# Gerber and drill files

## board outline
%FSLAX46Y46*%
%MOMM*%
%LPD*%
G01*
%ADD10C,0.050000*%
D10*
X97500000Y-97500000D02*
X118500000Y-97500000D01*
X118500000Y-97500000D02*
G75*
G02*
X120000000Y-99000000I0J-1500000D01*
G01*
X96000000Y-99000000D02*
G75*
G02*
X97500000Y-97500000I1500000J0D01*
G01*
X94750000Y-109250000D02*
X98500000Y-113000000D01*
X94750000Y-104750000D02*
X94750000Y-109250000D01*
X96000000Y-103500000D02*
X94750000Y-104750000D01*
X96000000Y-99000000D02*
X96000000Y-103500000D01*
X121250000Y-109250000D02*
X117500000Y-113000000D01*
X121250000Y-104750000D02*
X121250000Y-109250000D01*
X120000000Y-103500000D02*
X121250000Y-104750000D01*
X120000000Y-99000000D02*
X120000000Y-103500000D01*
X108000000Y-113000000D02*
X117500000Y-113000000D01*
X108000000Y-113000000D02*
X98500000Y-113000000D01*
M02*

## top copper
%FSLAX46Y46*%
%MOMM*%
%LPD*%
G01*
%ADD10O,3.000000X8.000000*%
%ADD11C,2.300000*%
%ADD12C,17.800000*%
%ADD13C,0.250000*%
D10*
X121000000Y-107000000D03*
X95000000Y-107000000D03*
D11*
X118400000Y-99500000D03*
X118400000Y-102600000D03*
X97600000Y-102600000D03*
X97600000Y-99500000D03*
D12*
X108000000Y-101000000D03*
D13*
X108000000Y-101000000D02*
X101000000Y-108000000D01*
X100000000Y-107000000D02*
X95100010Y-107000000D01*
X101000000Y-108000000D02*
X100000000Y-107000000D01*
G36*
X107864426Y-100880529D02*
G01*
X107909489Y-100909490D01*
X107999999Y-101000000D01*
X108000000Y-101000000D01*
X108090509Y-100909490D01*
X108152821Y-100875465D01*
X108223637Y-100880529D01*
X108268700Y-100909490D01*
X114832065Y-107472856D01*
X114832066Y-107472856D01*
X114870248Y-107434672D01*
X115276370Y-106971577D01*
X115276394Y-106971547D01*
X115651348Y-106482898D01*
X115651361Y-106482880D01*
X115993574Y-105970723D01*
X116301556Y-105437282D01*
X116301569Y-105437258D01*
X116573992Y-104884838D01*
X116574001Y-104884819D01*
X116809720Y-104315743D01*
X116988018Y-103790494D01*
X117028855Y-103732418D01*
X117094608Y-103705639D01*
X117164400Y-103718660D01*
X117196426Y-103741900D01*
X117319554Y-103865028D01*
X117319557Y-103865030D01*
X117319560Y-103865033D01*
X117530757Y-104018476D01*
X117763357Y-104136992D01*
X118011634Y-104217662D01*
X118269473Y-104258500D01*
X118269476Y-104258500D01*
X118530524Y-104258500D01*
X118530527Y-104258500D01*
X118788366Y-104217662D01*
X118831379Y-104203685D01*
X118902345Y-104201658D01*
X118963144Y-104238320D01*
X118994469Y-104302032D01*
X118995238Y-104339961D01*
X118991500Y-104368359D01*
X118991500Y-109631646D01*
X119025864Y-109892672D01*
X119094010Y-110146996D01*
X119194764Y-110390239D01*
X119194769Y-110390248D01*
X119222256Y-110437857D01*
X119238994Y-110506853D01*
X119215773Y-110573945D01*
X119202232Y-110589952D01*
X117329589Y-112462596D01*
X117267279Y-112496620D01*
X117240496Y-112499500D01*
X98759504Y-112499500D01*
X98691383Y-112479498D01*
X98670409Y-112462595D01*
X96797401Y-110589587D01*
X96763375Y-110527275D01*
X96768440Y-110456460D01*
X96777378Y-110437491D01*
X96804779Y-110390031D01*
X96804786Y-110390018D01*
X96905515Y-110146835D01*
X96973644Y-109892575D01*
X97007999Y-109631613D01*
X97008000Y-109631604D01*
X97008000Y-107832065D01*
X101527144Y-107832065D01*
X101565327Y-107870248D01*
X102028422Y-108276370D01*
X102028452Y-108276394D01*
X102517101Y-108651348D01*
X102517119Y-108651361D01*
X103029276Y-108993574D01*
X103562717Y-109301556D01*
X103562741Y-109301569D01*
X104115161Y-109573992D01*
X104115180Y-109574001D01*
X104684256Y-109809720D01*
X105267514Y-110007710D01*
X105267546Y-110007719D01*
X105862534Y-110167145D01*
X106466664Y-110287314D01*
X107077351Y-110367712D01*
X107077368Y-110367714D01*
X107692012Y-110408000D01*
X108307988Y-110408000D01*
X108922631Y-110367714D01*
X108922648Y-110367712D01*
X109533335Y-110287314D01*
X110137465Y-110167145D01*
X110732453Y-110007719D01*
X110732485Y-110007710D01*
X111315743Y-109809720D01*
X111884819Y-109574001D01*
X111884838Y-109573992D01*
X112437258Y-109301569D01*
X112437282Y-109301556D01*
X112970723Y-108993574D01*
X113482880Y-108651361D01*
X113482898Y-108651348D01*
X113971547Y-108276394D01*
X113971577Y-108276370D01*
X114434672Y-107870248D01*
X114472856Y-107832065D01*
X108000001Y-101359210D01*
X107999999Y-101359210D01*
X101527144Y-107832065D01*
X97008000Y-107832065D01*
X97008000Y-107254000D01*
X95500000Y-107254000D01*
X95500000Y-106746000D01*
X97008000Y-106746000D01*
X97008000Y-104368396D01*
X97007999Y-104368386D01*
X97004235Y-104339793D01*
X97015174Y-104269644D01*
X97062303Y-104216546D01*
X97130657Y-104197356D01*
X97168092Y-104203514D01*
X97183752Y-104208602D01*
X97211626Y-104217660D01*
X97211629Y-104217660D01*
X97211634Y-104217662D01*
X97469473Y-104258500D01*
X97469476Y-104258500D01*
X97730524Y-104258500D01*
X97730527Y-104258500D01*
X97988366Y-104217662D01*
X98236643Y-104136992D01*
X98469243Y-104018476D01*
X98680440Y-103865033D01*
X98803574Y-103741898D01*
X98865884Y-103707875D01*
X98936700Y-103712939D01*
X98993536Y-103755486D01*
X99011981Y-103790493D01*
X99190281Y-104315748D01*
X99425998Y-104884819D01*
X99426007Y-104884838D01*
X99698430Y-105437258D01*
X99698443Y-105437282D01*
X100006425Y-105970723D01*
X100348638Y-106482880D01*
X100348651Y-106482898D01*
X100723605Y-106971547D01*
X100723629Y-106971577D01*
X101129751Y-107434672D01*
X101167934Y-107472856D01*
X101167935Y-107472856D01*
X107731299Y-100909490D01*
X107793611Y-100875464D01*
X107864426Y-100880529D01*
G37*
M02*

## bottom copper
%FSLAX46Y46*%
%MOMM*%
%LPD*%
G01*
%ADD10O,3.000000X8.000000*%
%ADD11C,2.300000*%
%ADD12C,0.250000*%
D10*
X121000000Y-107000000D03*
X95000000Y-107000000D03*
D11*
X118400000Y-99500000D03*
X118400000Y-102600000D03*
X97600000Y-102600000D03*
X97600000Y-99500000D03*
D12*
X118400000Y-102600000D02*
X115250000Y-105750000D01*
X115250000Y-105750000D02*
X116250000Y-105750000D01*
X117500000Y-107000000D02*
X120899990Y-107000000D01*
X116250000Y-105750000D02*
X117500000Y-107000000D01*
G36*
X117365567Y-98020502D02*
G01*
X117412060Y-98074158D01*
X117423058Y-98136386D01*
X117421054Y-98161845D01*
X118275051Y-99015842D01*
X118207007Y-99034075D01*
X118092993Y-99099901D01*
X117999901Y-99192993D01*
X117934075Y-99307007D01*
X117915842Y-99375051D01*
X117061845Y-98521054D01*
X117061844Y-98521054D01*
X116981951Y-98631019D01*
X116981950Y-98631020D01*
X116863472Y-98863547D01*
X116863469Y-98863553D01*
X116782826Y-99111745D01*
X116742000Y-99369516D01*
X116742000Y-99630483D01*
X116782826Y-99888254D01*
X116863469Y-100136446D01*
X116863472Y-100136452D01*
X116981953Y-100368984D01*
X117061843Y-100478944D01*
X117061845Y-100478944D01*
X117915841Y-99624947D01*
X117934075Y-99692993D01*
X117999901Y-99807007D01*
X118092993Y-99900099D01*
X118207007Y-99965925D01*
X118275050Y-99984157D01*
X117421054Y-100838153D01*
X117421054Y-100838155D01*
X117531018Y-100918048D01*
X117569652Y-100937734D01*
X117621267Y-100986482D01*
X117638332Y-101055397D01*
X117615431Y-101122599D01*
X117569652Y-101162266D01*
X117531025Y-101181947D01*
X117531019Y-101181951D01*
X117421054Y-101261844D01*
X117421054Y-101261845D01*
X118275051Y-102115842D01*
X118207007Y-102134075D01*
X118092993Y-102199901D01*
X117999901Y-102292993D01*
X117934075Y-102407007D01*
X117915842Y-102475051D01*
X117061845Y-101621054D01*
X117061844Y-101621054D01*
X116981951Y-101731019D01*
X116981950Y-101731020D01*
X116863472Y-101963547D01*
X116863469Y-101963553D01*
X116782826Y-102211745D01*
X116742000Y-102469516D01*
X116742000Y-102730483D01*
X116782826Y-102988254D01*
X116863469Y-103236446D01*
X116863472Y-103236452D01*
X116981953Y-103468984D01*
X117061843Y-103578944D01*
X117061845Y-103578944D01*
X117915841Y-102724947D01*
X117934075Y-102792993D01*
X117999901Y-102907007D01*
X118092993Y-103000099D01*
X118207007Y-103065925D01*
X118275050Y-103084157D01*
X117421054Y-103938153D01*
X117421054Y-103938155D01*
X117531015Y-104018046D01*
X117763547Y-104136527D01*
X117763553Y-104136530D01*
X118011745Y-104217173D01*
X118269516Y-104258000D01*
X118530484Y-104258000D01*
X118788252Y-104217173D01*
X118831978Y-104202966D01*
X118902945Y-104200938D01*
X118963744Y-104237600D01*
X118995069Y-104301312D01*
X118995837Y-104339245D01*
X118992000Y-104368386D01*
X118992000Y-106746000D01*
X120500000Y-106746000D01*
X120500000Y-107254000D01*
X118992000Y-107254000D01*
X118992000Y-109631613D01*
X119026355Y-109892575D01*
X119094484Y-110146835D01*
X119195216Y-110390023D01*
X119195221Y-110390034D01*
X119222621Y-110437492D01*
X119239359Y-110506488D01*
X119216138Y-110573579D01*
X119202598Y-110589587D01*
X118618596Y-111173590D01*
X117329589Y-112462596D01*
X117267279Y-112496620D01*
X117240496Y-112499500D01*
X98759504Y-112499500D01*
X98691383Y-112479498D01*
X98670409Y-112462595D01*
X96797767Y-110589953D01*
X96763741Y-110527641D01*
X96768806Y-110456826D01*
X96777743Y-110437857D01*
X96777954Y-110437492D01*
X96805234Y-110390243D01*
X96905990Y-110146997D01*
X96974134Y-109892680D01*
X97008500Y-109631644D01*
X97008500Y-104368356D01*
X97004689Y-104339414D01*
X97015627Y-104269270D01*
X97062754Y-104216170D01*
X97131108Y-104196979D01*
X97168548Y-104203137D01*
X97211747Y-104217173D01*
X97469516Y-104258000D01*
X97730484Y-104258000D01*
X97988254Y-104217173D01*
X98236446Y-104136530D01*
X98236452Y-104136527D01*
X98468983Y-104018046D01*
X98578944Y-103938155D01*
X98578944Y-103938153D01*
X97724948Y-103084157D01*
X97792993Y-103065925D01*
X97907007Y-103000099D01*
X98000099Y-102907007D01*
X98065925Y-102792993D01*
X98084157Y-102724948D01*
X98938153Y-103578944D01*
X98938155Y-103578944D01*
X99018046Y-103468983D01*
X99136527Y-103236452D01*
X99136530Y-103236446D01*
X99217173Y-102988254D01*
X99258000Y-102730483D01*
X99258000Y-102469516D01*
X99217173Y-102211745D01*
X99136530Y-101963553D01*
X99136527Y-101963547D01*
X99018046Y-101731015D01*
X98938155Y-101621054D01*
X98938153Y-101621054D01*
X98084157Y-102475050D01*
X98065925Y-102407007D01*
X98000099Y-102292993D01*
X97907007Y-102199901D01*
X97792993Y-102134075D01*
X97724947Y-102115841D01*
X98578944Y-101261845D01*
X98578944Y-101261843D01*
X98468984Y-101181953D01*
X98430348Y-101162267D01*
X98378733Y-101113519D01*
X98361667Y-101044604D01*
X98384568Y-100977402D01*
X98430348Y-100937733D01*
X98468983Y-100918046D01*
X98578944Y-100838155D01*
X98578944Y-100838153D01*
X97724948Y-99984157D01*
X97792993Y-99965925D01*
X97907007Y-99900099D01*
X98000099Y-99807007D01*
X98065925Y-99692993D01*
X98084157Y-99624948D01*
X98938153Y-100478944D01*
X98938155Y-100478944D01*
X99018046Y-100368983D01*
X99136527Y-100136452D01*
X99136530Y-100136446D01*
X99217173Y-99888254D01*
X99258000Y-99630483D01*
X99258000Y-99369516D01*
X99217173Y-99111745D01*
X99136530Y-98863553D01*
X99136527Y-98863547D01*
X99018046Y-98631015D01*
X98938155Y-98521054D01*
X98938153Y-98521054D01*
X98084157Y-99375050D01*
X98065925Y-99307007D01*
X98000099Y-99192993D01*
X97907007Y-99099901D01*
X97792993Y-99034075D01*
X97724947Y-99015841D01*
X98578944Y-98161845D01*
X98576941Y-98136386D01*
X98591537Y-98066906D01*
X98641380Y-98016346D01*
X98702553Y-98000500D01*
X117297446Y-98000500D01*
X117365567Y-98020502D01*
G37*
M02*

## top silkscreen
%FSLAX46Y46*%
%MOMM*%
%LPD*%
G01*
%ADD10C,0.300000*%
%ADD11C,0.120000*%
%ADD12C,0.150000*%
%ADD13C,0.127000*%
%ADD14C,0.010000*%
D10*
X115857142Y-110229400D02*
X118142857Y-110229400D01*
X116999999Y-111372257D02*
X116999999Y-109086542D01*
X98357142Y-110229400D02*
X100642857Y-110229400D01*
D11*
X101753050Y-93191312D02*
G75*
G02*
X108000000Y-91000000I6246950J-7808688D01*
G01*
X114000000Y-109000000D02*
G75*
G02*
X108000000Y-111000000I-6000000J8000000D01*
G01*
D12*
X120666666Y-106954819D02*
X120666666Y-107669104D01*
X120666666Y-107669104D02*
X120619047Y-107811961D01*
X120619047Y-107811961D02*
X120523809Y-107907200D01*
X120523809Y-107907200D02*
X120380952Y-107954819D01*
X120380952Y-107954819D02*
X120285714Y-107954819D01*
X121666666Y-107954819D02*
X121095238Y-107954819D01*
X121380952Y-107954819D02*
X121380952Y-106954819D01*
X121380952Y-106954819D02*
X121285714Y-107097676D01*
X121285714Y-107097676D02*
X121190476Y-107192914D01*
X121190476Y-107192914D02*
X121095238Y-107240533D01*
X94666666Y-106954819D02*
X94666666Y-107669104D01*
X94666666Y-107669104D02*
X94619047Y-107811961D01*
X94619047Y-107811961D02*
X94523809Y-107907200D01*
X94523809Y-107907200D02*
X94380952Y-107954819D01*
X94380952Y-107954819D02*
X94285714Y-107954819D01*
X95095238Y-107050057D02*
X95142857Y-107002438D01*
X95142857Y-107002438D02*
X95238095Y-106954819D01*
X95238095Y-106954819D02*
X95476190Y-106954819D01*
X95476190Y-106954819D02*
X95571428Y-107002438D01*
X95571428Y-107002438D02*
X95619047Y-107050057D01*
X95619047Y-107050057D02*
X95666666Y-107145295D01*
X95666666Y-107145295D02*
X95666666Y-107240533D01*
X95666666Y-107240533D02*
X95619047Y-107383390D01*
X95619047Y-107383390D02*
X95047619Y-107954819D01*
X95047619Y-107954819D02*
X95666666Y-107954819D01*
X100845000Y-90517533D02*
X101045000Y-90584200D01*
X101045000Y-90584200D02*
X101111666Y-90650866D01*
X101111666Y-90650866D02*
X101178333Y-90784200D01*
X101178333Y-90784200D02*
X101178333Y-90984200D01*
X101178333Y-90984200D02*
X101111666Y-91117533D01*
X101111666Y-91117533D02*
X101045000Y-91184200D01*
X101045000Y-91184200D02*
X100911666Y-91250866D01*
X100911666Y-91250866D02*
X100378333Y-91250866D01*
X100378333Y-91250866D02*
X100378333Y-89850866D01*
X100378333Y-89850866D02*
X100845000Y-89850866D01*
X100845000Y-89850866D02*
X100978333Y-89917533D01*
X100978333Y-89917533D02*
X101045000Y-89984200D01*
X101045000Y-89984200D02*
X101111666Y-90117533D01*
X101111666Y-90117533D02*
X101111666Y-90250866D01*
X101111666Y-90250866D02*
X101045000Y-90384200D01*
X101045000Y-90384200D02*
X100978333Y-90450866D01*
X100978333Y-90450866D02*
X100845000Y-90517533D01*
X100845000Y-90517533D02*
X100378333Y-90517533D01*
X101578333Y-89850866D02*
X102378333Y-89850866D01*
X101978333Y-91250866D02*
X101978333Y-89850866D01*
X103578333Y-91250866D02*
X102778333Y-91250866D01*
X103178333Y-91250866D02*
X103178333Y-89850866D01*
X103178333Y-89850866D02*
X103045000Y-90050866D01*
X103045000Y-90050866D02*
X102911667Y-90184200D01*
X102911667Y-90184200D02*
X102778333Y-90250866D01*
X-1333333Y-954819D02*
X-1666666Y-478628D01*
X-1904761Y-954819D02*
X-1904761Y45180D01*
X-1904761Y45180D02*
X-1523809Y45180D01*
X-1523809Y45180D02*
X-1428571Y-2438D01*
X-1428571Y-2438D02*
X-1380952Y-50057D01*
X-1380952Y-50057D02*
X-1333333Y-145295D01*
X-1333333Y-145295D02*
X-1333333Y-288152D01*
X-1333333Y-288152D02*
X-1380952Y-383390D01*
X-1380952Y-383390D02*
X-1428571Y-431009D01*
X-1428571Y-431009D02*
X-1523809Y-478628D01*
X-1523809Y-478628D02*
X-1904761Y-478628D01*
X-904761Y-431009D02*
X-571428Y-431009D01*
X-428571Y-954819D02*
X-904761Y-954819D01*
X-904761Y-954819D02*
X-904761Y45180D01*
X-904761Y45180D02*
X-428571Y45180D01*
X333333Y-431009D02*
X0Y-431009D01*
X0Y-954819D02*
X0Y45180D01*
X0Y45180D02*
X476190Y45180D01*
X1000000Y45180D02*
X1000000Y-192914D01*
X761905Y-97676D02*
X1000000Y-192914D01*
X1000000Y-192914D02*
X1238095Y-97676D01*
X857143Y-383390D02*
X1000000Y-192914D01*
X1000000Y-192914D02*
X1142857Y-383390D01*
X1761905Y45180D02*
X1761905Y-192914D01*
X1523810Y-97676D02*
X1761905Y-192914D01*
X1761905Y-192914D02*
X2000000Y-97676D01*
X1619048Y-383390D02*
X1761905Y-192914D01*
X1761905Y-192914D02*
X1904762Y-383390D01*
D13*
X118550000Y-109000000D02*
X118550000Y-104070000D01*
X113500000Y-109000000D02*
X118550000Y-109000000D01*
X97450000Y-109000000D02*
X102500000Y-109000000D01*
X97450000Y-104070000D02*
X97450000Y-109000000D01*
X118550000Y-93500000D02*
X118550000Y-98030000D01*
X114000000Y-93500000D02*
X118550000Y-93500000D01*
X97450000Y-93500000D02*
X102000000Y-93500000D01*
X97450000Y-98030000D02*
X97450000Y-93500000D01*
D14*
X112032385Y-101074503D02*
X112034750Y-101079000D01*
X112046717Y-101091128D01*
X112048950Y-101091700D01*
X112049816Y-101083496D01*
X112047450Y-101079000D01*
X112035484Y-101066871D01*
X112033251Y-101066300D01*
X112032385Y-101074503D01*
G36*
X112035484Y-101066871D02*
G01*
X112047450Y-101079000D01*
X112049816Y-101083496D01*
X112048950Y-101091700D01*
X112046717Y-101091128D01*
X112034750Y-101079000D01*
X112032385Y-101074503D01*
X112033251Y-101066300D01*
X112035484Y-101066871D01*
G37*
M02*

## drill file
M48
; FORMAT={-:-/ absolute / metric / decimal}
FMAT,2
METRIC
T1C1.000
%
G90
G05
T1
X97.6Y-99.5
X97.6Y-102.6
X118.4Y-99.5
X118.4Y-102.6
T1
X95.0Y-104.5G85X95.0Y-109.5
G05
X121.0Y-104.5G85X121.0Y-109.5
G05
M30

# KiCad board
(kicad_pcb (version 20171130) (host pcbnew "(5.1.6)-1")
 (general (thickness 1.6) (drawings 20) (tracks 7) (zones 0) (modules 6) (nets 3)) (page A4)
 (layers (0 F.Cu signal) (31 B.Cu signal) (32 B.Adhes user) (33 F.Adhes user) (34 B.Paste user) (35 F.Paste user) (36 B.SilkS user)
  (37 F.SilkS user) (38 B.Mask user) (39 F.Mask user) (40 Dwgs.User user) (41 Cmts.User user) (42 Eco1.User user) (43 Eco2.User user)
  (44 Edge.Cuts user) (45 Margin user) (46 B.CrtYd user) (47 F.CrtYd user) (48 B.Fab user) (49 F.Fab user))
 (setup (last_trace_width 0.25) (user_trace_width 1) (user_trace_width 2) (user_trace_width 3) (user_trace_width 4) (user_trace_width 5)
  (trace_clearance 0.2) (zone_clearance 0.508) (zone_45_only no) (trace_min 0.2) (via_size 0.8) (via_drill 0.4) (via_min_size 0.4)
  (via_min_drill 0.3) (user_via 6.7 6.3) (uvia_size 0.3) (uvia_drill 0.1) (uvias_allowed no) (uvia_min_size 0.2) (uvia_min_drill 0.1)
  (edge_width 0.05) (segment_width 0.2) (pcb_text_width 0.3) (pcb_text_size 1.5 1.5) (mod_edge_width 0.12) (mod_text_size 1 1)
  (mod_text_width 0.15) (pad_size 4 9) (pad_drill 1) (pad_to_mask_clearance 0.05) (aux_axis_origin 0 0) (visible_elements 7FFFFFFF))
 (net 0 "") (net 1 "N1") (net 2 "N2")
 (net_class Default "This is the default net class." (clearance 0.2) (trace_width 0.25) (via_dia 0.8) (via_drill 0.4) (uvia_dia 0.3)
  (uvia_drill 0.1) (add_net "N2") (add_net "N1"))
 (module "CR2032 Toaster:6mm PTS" (layer F.Cu) (at 121 107)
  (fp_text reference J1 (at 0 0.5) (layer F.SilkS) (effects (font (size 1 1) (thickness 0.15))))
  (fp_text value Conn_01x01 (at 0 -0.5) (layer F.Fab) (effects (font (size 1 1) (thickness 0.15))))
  (pad 1 thru_hole oval (at 0 0) (size 3 8) (drill oval 1 6) (layers *.Cu *.Mask) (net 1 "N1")))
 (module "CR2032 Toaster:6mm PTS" (layer F.Cu) (at 95 107)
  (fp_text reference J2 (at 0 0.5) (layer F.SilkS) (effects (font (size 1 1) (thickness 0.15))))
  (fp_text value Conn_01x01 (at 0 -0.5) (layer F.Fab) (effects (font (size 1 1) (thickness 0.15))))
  (pad 1 thru_hole oval (at 0 0) (size 3 8) (drill oval 1 6) (layers *.Cu *.Mask) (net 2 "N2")))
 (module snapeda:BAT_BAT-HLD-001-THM (layer F.Cu) (at 108 101)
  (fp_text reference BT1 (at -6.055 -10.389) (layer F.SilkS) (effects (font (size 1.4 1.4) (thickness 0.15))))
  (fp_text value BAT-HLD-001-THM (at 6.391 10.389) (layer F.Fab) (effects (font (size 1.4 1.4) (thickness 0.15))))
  (fp_line (start 10.55 8) (end 10.55 3.07) (layer F.SilkS) (width 0.127))
  (fp_line (start 5.5 8) (end 10.55 8) (layer F.SilkS) (width 0.127))
  (fp_line (start -10.55 8) (end -5.5 8) (layer F.SilkS) (width 0.127))
  (fp_line (start -10.55 3.07) (end -10.55 8) (layer F.SilkS) (width 0.127))
  (fp_line (start 10.55 -7.5) (end 10.55 -2.97) (layer F.SilkS) (width 0.127))
  (fp_line (start 6 -7.5) (end 10.55 -7.5) (layer F.SilkS) (width 0.127))
  (fp_line (start -10.55 -7.5) (end -6 -7.5) (layer F.SilkS) (width 0.127))
  (fp_line (start -10.55 -2.97) (end -10.55 -7.5) (layer F.SilkS) (width 0.127))
  (pad P4 thru_hole circle (at 10.4 -1.5) (size 2.3 2.3) (drill 1) (layers *.Cu *.Mask) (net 1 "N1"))
  (pad P3 thru_hole circle (at 10.4 1.6) (size 2.3 2.3) (drill 1) (layers *.Cu *.Mask) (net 1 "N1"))
  (pad P2 thru_hole circle (at -10.4 1.6) (size 2.3 2.3) (drill 1) (layers *.Cu *.Mask) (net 1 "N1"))
  (pad P1 thru_hole circle (at -10.4 -1.5) (size 2.3 2.3) (drill 1) (layers *.Cu *.Mask) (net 1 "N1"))
  (pad N smd circle (at 0 0) (size 17.8 17.8) (layers F.Cu F.Mask) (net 2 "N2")))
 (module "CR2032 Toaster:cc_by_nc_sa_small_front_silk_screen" (layer B.Cu) (at 108 110 180)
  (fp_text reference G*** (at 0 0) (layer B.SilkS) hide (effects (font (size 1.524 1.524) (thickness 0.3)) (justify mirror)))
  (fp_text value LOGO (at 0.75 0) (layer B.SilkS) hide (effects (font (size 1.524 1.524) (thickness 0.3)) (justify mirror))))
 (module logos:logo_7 (layer F.Cu) (at 113.4 103)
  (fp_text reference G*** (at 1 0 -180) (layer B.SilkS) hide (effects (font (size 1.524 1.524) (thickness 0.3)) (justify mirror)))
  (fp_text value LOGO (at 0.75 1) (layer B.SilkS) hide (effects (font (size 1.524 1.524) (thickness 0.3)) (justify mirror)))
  (fp_poly
   (pts (xy -1.367615 -1.925497) (xy -1.36525 -1.921) (xy -1.353283 -1.908872) (xy -1.35105 -1.9083) (xy -1.350184 -1.916504)
    (xy -1.35255 -1.921) (xy -1.364516 -1.933129) (xy -1.366749 -1.9337) (xy -1.367615 -1.925497))
   (layer F.SilkS) (width 0.01)))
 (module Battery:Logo (layer F.Cu) (at 0 0)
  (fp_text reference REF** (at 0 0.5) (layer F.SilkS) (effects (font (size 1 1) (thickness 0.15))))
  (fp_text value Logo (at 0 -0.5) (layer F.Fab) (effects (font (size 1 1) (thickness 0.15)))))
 (gr_line (start 97.5 97.5) (end 118.5 97.5) (layer Edge.Cuts) (width 0.05))
 (gr_arc (start 118.5 99) (end 120 99) (angle -90) (layer Edge.Cuts) (width 0.05))
 (gr_arc (start 97.5 99) (end 97.5 97.5) (angle -90) (layer Edge.Cuts) (width 0.05))
 (gr_line (start 94.75 109.25) (end 98.5 113) (layer Edge.Cuts) (width 0.05))
 (gr_line (start 94.75 104.75) (end 94.75 109.25) (layer Edge.Cuts) (width 0.05))
 (gr_line (start 96 103.5) (end 94.75 104.75) (layer Edge.Cuts) (width 0.05))
 (gr_line (start 96 99) (end 96 103.5) (layer Edge.Cuts) (width 0.05))
 (gr_line (start 121.25 109.25) (end 117.5 113) (layer Edge.Cuts) (width 0.05))
 (gr_line (start 121.25 104.75) (end 121.25 109.25) (layer Edge.Cuts) (width 0.05))
 (gr_line (start 120 103.5) (end 121.25 104.75) (layer Edge.Cuts) (width 0.05))
 (gr_line (start 120 99) (end 120 103.5) (layer Edge.Cuts) (width 0.05))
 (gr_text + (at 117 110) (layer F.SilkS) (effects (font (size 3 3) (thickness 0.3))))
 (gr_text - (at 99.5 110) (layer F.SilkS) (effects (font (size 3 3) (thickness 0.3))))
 (gr_line (start 108 113) (end 117.5 113) (layer Edge.Cuts) (width 0.05))
 (gr_line (start 108 113) (end 98.5 113) (layer Edge.Cuts) (width 0.05))
 (gr_arc (start 108 101) (end 108 91) (angle -38.65980825) (layer F.SilkS) (width 0.12))
 (gr_arc (start 108 101) (end 108 111) (angle -36.86989765) (layer F.SilkS) (width 0.12))
 (segment (start 118.4 102.6) (end 115.25 105.75) (width 0.25) (layer B.Cu) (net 1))
 (segment (start 115.25 105.75) (end 116.25 105.75) (width 0.25) (layer B.Cu) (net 1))
 (segment (start 117.5 107) (end 120.89999 107) (width 0.25) (layer B.Cu) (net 1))
 (segment (start 116.25 105.75) (end 117.5 107) (width 0.25) (layer B.Cu) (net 1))
 (segment (start 108 101) (end 101 108) (width 0.25) (layer F.Cu) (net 2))
 (segment (start 100 107) (end 95.10001 107) (width 0.25) (layer F.Cu) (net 2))
 (segment (start 101 108) (end 100 107) (width 0.25) (layer F.Cu) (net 2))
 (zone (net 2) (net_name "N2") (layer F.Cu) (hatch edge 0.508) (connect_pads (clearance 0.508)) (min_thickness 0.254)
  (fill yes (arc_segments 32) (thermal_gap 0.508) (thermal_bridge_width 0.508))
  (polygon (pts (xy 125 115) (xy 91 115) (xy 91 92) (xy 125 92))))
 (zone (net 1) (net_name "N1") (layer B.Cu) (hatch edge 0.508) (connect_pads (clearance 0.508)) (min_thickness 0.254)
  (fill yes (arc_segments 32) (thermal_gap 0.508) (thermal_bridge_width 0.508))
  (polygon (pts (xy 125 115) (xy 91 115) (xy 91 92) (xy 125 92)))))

